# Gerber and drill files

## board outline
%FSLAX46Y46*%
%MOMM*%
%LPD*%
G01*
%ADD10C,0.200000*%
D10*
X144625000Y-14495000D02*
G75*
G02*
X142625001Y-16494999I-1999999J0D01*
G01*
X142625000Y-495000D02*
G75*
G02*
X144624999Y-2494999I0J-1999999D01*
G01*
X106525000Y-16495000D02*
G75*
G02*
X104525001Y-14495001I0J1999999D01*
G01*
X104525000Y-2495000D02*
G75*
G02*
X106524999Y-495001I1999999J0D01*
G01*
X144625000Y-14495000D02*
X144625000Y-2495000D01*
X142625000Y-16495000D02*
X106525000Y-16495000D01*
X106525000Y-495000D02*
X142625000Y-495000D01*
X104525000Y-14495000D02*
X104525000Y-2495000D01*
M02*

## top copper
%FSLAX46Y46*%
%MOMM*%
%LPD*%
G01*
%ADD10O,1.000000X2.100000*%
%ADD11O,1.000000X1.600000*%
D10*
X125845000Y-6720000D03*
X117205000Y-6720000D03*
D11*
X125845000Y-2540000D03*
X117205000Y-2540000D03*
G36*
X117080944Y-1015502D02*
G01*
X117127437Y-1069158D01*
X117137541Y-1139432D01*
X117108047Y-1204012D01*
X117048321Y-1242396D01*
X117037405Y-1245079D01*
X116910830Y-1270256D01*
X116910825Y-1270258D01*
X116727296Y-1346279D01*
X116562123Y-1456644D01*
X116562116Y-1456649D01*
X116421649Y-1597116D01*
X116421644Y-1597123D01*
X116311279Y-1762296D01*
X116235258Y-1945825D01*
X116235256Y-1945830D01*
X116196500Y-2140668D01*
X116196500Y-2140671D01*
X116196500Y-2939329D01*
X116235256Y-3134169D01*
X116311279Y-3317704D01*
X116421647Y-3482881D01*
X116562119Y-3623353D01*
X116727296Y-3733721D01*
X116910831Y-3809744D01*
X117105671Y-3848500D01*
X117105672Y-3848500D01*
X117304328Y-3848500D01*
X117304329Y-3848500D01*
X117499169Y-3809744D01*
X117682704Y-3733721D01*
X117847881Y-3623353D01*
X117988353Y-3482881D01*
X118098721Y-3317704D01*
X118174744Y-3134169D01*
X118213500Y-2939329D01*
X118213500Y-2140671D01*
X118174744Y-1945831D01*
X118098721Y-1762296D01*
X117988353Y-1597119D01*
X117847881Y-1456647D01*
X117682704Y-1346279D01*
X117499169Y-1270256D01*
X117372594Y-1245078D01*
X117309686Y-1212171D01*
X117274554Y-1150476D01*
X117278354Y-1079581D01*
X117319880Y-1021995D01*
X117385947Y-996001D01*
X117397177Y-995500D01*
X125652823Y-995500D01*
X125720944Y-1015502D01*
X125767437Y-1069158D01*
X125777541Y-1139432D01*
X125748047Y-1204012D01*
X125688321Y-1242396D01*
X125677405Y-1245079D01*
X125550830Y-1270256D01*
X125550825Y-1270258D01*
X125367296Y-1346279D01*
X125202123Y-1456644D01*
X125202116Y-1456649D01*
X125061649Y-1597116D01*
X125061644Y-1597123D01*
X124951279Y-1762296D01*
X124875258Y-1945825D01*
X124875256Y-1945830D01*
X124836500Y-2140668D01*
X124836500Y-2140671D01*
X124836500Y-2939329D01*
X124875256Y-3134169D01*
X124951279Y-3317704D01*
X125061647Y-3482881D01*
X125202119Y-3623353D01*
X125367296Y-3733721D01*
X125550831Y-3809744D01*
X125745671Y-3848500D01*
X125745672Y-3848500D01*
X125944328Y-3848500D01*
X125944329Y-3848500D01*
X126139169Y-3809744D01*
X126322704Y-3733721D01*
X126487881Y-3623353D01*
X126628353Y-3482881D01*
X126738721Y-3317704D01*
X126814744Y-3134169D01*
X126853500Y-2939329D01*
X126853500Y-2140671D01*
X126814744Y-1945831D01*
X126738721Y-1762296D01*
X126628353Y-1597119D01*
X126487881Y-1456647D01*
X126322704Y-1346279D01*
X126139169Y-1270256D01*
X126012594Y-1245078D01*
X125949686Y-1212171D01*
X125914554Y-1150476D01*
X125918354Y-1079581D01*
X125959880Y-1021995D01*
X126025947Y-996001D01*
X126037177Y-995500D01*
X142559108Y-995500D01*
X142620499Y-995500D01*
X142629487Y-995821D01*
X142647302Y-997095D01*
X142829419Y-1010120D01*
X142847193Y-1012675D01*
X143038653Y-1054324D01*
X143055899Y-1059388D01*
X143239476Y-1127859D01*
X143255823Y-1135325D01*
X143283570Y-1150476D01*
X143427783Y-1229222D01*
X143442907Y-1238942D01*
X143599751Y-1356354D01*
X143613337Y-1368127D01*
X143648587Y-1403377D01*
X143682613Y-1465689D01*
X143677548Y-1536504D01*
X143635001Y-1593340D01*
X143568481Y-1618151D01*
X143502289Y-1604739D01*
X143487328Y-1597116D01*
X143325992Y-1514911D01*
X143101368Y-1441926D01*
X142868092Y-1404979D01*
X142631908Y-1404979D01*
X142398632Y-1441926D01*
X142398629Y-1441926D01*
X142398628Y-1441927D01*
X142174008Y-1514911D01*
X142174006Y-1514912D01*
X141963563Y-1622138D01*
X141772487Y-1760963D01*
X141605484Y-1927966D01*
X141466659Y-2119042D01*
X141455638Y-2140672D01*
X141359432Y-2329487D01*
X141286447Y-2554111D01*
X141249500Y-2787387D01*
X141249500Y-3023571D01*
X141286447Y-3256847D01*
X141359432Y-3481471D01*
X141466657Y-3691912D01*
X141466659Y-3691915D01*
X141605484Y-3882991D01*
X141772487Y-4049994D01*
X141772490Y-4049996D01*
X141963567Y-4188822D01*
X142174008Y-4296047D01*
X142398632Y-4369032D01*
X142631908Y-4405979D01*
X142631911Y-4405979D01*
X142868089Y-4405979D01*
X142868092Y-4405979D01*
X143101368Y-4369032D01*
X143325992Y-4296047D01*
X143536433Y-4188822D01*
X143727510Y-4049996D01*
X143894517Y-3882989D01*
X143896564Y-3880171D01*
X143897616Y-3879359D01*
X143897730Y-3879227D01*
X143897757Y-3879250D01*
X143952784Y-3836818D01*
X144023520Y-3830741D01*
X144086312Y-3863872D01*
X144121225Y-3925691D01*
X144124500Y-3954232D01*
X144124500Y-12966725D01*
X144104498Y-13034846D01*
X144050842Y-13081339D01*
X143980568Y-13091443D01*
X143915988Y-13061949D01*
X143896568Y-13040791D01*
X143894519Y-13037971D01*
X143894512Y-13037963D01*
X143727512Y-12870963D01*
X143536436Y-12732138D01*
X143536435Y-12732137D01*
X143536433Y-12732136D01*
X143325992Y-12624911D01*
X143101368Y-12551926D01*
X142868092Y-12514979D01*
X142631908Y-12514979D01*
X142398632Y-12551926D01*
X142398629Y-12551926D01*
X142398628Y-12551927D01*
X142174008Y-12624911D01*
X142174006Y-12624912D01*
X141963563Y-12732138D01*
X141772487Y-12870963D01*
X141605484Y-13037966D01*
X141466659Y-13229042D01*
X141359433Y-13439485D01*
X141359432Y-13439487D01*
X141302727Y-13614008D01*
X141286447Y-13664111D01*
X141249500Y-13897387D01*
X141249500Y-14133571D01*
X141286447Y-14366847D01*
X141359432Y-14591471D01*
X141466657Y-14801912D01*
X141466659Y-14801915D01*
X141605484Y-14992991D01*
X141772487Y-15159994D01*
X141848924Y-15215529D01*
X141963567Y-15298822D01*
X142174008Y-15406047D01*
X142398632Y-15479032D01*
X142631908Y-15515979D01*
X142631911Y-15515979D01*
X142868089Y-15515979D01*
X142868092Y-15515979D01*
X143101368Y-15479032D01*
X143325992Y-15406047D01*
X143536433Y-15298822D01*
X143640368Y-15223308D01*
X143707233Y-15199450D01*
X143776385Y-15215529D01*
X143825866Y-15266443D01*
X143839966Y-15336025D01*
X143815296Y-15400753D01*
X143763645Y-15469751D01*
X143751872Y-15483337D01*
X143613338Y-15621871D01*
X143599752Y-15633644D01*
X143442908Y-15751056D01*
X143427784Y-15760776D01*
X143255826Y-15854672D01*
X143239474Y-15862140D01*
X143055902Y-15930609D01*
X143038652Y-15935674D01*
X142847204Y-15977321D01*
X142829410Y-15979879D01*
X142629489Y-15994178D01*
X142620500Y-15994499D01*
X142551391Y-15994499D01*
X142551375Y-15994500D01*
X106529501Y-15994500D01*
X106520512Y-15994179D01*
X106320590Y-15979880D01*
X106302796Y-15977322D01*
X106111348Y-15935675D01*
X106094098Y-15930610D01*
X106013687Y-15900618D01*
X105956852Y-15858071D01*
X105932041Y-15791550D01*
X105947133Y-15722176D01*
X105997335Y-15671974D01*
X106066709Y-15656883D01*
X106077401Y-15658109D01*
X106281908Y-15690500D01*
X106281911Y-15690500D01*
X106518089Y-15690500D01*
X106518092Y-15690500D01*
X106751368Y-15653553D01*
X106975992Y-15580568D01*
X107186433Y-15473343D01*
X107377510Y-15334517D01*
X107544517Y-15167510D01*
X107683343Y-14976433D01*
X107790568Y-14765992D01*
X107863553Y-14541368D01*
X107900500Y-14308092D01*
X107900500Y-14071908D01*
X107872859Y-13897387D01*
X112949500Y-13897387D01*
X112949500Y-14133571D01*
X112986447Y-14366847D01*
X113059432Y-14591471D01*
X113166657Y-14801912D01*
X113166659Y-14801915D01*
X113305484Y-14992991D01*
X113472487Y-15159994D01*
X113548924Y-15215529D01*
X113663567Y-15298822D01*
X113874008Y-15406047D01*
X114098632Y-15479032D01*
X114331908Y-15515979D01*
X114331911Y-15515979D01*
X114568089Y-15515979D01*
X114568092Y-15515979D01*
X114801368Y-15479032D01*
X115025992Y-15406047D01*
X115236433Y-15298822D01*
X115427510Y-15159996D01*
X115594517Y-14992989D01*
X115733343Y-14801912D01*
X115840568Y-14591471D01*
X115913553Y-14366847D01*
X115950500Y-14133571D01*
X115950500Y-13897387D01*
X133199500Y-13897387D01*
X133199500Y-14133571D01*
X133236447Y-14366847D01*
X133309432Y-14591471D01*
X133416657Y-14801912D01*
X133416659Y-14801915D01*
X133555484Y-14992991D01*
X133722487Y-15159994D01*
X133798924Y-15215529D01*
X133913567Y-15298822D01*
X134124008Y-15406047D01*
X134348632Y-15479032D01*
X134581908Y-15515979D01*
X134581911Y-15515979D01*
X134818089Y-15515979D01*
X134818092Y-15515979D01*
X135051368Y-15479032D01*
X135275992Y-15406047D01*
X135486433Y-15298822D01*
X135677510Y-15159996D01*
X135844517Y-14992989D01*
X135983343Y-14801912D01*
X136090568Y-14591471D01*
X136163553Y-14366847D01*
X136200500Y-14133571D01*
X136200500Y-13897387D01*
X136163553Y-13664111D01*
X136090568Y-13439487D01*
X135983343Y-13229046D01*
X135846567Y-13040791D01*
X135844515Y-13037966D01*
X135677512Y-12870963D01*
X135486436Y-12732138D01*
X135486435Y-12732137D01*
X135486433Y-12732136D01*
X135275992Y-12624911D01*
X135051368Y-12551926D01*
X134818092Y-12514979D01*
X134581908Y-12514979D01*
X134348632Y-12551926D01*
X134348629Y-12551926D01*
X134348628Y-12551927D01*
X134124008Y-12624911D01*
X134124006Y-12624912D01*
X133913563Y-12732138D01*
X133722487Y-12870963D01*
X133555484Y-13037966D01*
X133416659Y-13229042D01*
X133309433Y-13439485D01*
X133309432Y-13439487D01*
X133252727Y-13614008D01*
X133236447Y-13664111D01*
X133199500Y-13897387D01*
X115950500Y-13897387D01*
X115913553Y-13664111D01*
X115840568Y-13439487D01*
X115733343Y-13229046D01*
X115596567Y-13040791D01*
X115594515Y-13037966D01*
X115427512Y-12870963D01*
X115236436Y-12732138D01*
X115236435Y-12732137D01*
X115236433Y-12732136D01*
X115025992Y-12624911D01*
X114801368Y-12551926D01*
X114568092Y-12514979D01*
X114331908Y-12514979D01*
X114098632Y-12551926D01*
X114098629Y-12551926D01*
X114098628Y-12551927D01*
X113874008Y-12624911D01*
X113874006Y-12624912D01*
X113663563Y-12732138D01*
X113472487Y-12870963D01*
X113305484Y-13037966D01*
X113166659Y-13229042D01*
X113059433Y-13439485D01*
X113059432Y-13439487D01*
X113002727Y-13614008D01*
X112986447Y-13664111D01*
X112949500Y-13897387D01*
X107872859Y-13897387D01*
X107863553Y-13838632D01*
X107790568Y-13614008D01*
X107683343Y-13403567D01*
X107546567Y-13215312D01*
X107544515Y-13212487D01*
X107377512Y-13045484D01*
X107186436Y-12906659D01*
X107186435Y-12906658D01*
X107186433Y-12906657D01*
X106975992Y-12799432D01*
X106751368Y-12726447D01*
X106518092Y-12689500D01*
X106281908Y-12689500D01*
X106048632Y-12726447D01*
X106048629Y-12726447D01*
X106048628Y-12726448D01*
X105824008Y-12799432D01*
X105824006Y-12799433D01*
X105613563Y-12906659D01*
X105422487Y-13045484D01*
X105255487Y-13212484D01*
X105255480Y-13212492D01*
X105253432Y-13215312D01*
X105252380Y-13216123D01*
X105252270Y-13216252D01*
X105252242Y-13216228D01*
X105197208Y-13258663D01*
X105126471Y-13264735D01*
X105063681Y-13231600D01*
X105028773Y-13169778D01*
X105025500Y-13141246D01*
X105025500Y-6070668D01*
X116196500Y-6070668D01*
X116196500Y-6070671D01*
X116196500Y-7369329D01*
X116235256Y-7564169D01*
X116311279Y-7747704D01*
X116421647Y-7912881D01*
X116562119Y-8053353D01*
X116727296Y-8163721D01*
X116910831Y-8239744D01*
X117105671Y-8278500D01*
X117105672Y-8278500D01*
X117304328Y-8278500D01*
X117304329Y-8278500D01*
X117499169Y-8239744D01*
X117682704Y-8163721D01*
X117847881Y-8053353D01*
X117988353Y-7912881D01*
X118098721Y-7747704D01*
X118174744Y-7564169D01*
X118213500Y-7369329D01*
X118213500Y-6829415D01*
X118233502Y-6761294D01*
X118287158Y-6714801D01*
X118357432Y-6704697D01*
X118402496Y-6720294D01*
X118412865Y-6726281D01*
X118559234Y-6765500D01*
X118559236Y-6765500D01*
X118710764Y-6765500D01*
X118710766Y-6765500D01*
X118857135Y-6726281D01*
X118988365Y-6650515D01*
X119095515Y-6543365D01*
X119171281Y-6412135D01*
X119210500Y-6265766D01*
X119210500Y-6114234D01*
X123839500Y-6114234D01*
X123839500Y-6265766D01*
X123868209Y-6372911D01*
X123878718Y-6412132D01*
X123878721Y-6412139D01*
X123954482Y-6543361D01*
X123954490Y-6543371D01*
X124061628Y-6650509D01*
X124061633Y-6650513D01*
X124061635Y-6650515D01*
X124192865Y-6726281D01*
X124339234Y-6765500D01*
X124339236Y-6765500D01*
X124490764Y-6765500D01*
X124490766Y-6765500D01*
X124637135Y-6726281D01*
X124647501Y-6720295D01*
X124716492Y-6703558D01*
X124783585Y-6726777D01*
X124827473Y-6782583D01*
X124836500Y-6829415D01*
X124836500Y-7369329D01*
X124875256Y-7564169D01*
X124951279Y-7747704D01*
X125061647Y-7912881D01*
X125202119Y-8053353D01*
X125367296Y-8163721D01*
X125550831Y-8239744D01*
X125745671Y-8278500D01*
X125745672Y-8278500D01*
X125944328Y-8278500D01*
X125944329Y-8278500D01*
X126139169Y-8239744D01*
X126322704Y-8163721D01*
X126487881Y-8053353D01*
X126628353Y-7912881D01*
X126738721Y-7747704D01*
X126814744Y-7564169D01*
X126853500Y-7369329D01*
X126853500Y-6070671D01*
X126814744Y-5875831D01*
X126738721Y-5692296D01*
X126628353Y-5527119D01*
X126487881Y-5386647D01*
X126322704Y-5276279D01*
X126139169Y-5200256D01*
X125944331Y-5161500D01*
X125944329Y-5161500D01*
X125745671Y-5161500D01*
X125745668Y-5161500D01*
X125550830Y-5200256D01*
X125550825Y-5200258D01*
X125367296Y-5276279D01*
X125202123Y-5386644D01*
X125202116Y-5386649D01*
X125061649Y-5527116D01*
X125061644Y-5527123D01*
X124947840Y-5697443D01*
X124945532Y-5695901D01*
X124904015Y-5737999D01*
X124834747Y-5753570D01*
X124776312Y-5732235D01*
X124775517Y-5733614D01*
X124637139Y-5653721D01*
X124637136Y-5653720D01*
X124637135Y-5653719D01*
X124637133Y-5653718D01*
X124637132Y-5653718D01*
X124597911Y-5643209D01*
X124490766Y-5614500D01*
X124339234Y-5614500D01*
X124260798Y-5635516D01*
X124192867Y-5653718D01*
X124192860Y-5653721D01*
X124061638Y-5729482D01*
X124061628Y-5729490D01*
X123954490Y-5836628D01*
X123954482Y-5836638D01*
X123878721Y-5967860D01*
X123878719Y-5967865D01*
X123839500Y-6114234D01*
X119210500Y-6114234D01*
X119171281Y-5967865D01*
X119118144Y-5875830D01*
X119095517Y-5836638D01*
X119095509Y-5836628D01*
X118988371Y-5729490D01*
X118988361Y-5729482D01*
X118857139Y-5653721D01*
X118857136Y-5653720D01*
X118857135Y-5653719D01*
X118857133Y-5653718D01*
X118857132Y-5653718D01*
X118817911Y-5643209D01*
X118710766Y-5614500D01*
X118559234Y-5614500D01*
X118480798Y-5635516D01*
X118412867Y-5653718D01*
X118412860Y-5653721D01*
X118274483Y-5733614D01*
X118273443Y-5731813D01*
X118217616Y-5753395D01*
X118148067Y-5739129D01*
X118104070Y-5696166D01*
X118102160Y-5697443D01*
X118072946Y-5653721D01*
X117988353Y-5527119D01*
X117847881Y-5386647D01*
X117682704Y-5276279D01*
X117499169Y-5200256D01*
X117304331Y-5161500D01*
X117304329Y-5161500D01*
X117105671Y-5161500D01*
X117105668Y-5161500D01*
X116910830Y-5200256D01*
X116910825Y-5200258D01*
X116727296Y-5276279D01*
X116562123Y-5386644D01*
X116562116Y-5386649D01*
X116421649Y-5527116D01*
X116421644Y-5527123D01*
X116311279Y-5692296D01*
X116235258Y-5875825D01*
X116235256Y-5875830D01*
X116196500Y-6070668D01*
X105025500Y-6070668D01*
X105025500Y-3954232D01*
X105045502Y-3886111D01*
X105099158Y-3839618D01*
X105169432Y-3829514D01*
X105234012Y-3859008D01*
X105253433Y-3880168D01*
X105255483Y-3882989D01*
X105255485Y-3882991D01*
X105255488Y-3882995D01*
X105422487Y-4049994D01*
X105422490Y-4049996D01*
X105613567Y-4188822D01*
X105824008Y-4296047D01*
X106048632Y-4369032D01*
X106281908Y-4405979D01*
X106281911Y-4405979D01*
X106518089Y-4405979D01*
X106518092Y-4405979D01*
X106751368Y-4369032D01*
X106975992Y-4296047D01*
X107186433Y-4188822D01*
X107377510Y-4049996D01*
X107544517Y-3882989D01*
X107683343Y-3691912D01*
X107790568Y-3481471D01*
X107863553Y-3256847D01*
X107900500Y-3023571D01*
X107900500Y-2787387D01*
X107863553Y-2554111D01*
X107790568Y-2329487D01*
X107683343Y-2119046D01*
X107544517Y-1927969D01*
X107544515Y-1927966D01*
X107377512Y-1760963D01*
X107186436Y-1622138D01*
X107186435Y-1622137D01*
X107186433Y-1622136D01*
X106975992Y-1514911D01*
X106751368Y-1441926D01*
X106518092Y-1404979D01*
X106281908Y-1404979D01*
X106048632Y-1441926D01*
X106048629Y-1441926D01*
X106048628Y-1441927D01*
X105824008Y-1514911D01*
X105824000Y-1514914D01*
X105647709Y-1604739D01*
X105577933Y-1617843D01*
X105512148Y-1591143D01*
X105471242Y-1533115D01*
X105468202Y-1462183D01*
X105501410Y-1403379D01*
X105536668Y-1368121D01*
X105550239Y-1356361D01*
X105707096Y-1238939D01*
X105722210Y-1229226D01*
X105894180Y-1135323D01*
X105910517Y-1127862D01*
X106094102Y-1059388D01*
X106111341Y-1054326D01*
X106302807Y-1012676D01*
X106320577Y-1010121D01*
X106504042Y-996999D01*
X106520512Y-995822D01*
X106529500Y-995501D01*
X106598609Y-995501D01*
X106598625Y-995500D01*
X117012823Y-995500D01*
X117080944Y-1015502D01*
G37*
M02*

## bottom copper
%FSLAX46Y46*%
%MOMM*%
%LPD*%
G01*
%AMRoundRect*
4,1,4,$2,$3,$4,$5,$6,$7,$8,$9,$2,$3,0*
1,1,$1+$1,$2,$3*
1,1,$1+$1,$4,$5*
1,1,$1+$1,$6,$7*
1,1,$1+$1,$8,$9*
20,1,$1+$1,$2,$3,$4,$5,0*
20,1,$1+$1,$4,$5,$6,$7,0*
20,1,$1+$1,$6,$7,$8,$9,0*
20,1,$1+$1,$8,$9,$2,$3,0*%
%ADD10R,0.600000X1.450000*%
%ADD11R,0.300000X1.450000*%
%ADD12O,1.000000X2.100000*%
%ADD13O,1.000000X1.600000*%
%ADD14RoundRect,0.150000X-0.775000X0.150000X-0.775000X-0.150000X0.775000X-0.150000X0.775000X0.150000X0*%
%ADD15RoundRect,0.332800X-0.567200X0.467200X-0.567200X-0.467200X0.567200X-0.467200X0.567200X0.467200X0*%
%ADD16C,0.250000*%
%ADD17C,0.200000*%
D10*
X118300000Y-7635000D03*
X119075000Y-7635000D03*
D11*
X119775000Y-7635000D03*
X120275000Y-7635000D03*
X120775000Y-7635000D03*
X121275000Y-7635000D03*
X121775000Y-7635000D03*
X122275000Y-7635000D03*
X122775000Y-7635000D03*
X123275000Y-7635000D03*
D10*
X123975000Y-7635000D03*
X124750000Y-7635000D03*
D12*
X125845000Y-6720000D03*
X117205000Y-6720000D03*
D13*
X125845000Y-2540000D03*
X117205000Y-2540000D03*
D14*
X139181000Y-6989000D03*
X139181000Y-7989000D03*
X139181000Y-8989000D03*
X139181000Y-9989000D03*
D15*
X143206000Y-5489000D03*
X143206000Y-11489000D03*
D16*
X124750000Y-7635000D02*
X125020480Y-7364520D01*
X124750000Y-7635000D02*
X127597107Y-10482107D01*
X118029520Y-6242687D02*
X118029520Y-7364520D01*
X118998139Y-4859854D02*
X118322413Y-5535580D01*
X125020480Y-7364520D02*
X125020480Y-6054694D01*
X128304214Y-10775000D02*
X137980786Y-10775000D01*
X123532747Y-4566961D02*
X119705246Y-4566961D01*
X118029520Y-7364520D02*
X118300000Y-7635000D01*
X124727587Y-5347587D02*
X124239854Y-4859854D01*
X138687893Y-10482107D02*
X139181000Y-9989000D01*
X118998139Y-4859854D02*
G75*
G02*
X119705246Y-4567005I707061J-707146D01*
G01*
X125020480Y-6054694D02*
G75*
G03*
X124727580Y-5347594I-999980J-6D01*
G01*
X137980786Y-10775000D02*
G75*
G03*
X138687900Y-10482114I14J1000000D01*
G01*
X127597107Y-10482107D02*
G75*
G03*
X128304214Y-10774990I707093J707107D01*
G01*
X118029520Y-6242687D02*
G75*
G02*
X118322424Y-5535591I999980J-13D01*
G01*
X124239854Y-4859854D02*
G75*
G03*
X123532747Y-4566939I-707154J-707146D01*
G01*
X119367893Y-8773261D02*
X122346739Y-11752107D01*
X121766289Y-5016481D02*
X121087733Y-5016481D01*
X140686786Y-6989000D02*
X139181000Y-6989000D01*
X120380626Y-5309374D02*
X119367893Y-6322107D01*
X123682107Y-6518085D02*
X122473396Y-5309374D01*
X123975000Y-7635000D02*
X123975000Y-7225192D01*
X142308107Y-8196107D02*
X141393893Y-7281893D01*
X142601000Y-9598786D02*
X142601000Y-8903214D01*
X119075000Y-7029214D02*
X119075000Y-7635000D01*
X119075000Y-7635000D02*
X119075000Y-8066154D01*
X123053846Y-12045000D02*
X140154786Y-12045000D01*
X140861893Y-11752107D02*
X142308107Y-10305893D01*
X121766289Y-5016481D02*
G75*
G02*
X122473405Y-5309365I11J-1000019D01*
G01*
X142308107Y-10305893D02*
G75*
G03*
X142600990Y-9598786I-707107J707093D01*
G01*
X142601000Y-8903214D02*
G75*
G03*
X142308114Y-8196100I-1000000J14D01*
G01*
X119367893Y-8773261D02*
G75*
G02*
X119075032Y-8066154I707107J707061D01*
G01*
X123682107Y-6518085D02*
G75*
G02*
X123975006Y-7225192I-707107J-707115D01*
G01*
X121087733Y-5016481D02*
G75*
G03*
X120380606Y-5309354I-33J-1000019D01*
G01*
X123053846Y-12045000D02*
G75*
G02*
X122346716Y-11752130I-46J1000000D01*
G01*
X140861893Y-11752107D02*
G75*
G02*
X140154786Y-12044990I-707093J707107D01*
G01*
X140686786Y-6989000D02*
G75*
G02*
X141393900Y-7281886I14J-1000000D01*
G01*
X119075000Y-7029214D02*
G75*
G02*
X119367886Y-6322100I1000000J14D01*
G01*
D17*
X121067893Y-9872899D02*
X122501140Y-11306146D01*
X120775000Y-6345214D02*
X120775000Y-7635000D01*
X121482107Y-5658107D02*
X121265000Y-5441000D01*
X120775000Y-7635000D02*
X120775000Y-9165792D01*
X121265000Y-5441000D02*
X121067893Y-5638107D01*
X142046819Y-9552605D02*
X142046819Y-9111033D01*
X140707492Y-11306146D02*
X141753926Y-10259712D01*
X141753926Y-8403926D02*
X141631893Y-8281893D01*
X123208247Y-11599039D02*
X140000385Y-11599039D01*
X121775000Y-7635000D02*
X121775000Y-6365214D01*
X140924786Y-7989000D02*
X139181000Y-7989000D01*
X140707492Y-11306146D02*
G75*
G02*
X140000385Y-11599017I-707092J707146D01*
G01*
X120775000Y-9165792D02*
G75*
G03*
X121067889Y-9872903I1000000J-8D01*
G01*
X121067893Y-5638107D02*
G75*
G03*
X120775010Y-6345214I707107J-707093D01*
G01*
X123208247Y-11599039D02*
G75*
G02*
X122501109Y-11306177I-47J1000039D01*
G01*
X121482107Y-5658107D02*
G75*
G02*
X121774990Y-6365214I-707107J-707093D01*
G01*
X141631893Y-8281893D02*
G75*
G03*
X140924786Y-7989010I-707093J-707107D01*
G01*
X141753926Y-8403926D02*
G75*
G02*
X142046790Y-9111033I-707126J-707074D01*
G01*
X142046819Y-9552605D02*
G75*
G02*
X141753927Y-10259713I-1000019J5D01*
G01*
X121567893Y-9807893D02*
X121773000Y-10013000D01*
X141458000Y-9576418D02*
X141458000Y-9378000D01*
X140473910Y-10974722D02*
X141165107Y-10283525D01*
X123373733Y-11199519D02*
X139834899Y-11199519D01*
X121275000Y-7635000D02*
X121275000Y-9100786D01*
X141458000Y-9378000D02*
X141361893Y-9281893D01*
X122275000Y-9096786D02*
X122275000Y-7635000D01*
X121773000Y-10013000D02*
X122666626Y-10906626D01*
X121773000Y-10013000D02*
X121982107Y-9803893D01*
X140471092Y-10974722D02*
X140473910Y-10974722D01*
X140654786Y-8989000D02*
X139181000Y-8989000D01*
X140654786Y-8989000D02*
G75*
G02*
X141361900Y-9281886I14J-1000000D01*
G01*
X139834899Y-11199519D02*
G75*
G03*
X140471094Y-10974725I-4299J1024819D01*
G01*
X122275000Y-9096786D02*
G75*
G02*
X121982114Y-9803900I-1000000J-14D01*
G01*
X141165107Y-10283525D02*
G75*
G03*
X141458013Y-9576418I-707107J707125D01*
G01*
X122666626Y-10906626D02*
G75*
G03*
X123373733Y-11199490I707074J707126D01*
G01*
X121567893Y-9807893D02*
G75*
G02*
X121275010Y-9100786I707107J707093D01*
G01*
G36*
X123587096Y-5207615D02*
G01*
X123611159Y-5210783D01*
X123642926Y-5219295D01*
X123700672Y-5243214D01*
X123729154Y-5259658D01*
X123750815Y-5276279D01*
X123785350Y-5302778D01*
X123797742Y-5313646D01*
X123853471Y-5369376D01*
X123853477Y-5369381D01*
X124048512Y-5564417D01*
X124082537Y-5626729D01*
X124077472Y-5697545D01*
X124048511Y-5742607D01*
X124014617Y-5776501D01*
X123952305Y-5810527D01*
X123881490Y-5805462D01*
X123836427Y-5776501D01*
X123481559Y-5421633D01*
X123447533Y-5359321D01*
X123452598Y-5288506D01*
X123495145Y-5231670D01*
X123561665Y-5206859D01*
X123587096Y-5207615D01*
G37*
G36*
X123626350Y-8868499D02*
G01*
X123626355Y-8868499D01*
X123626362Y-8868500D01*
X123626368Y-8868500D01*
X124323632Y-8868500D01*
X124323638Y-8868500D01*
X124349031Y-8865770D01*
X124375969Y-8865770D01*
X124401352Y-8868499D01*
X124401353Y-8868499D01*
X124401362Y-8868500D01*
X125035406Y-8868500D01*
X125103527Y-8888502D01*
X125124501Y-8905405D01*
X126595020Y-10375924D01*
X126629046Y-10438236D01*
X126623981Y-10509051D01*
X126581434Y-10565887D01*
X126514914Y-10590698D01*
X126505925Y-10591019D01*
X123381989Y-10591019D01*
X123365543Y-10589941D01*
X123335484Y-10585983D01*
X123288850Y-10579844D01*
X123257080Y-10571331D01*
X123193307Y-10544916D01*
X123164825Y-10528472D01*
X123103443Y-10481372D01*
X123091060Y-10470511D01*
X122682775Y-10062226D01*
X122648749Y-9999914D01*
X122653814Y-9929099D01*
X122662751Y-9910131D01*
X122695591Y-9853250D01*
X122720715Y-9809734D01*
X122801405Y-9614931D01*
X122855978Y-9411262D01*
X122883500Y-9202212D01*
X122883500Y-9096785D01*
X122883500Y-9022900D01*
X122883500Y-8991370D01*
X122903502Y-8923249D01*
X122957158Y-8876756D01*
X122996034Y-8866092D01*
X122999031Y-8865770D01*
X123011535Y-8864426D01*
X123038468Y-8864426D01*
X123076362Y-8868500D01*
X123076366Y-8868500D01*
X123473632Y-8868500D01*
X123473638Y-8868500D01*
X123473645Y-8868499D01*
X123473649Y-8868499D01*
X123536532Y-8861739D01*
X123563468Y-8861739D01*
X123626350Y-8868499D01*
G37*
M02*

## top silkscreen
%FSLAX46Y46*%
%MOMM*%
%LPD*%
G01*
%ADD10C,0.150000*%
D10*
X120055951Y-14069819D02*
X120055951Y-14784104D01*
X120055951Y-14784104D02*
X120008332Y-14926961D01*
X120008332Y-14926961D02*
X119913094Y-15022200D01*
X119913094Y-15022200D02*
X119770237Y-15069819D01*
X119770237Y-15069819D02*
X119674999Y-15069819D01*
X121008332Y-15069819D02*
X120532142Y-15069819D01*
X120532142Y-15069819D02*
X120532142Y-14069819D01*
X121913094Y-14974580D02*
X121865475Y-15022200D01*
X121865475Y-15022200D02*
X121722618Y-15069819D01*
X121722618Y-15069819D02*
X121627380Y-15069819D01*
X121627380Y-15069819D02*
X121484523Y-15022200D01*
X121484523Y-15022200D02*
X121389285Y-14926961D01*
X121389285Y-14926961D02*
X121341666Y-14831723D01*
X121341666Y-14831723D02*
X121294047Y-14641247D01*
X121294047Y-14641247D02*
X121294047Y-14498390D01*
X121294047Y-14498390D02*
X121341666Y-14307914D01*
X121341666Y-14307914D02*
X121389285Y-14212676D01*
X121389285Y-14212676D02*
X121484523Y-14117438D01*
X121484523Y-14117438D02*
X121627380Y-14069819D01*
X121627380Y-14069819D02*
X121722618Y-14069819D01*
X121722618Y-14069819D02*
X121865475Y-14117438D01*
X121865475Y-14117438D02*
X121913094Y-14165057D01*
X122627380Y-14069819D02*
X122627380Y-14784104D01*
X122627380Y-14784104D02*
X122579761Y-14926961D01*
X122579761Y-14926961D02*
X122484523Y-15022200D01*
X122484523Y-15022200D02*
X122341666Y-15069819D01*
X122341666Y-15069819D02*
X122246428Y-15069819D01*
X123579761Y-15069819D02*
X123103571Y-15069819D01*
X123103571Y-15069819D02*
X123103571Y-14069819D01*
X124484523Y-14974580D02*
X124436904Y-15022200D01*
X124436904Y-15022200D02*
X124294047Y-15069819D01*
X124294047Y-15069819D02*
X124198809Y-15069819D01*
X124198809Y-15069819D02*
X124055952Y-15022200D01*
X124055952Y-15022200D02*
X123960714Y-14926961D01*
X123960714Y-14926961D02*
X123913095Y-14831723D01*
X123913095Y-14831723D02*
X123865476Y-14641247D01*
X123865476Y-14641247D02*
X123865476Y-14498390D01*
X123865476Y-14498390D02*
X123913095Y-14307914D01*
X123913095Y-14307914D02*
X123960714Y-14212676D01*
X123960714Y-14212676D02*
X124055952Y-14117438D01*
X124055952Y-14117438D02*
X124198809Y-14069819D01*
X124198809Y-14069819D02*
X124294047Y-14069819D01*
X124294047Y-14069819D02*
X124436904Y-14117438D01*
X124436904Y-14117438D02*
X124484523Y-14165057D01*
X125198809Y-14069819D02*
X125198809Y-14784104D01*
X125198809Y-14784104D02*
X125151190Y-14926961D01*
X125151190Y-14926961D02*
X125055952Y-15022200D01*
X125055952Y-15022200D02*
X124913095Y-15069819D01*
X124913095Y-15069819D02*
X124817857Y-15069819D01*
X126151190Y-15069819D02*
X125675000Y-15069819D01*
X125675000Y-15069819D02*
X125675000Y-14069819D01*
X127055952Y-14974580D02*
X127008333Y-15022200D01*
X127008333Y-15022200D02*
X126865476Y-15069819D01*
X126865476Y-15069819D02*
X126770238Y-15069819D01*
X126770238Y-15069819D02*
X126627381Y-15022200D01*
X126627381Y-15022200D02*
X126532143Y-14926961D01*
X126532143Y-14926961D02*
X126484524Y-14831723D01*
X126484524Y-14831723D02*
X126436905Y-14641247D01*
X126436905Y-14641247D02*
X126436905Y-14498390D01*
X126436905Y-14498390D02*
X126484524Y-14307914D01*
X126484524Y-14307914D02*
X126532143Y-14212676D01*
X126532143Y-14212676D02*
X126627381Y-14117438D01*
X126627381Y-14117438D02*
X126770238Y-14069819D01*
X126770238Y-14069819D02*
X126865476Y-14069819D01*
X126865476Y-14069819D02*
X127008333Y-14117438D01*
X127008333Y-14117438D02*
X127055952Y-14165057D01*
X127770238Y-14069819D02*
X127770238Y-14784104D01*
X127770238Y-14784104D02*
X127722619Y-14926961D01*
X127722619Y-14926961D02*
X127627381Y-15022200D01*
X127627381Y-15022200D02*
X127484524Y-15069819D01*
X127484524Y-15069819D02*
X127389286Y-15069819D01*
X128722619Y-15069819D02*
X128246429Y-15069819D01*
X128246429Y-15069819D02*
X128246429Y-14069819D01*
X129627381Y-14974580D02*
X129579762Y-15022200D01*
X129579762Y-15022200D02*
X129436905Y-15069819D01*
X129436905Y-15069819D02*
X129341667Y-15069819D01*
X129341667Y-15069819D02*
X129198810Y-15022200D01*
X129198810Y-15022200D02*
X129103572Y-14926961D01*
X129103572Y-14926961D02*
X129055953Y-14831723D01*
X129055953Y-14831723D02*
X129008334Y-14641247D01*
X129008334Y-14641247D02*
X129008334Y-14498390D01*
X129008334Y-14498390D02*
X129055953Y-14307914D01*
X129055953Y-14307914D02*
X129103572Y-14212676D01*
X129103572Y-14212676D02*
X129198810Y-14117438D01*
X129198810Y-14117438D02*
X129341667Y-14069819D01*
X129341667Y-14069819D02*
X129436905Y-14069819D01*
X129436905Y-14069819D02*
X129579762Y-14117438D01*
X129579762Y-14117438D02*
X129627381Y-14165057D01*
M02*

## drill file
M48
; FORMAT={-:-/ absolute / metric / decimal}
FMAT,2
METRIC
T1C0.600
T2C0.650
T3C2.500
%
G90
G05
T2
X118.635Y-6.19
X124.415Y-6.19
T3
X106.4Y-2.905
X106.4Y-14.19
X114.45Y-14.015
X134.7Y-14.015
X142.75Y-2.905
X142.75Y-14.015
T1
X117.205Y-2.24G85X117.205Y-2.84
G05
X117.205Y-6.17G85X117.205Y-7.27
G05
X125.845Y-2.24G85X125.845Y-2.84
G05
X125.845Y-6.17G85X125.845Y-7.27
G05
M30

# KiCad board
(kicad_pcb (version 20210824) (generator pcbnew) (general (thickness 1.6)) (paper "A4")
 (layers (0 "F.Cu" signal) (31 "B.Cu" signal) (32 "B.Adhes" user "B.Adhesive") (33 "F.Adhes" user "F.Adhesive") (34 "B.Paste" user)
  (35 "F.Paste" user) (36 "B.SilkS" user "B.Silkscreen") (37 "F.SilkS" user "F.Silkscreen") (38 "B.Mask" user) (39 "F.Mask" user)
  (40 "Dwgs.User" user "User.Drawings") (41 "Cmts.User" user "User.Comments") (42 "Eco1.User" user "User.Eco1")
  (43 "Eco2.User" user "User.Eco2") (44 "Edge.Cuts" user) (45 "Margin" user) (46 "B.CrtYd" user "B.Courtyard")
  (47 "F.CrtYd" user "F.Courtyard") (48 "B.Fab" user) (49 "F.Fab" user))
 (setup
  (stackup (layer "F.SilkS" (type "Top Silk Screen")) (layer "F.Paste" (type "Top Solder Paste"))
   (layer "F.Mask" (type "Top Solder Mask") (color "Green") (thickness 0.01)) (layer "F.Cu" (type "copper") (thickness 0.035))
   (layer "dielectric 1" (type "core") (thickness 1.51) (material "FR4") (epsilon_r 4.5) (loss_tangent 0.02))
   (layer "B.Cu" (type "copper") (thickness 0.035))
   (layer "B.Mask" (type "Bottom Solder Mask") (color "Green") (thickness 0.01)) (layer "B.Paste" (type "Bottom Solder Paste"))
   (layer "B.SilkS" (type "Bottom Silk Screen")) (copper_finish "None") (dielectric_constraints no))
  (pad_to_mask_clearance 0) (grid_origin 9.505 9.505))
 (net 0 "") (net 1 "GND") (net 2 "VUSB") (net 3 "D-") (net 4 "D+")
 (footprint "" (layer "F.Cu") (at 136.255 14.205)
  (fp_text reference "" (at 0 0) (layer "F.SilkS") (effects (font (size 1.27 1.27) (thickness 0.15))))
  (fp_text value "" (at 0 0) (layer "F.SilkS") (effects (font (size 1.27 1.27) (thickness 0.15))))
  (pad "" np_thru_hole circle (at -1.555 -0.189521) (size 2.5 2.5) (drill 2.5) (layers F&B.Cu *.Mask)))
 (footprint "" (layer "F.Cu") (at 94.555 1.535)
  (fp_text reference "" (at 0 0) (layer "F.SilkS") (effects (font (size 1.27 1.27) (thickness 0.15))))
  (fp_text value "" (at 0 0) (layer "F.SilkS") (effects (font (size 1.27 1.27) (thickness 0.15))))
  (pad "" np_thru_hole circle (at 11.845 1.370479) (size 2.5 2.5) (drill 2.5) (layers F&B.Cu *.Mask)))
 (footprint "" (layer "F.Cu") (at 147.015 3.065)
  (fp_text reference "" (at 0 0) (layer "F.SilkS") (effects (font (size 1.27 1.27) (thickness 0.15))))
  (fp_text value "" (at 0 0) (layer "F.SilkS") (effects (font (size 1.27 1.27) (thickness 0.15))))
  (pad "" np_thru_hole circle (at -4.265 -0.159521) (size 2.5 2.5) (drill 2.5) (layers F&B.Cu *.Mask)))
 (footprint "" (layer "F.Cu") (at 94.295 7.445633)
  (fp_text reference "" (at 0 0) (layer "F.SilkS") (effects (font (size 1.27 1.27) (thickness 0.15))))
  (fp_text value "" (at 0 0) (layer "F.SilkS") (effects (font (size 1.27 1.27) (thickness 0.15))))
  (pad "" np_thru_hole circle (at 12.105 6.744367) (size 2.5 2.5) (drill 2.5) (layers F&B.Cu *.Mask)))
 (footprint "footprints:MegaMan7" (layer "F.Cu") (at 109.650838 8.415023)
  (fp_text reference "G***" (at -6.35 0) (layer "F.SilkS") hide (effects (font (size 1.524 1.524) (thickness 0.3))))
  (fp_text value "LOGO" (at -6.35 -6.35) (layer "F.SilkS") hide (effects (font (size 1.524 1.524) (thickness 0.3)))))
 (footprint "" (layer "F.Cu") (at 112.225 13.965)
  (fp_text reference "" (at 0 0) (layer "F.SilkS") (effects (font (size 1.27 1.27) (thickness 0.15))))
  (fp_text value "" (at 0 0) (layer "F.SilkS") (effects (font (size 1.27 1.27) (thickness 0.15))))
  (pad "" np_thru_hole circle (at 2.225 0.050479) (size 2.5 2.5) (drill 2.5) (layers F&B.Cu *.Mask)))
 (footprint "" (layer "F.Cu") (at 130.75 14.19)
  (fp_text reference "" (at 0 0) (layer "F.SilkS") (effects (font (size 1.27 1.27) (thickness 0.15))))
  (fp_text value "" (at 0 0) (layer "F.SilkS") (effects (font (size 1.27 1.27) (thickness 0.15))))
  (pad "" np_thru_hole circle (at 12 -0.174521) (size 2.5 2.5) (drill 2.5) (layers F&B.Cu *.Mask)))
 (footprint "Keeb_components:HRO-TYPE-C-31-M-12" (layer "B.Cu") (at 121.525 -0.06)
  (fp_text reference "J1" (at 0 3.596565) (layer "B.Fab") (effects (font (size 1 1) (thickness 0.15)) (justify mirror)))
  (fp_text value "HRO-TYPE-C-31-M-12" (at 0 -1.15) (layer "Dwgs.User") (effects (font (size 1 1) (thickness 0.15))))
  (pad "" np_thru_hole circle locked (at -2.89 6.25) (size 0.65 0.65) (drill 0.65) (layers *.Cu *.Mask))
  (pad "" np_thru_hole circle locked (at 2.89 6.25) (size 0.65 0.65) (drill 0.65) (layers *.Cu *.Mask))
  (pad "1" smd rect locked (at -3.225 7.695) (size 0.6 1.45) (layers "B.Cu" "B.Paste" "B.Mask") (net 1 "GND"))
  (pad "2" smd rect locked (at -2.45 7.695) (size 0.6 1.45) (layers "B.Cu" "B.Paste" "B.Mask") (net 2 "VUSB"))
  (pad "3" smd rect locked (at -1.75 7.695) (size 0.3 1.45) (layers "B.Cu" "B.Paste" "B.Mask"))
  (pad "4" smd rect locked (at -1.25 7.695) (size 0.3 1.45) (layers "B.Cu" "B.Paste" "B.Mask"))
  (pad "5" smd rect locked (at -0.75 7.695) (size 0.3 1.45) (layers "B.Cu" "B.Paste" "B.Mask") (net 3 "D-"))
  (pad "6" smd rect locked (at -0.25 7.695) (size 0.3 1.45) (layers "B.Cu" "B.Paste" "B.Mask") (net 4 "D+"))
  (pad "7" smd rect locked (at 0.25 7.695) (size 0.3 1.45) (layers "B.Cu" "B.Paste" "B.Mask") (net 3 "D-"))
  (pad "8" smd rect locked (at 0.75 7.695) (size 0.3 1.45) (layers "B.Cu" "B.Paste" "B.Mask") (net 4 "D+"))
  (pad "9" smd rect locked (at 1.25 7.695) (size 0.3 1.45) (layers "B.Cu" "B.Paste" "B.Mask"))
  (pad "10" smd rect locked (at 1.75 7.695) (size 0.3 1.45) (layers "B.Cu" "B.Paste" "B.Mask"))
  (pad "11" smd rect locked (at 2.45 7.695) (size 0.6 1.45) (layers "B.Cu" "B.Paste" "B.Mask") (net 2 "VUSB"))
  (pad "12" smd rect locked (at 3.225 7.695) (size 0.6 1.45) (layers "B.Cu" "B.Paste" "B.Mask") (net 1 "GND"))
  (pad "13" thru_hole oval locked (at 4.32 6.78) (size 1 2.1) (drill oval 0.6 1.7) (layers *.Cu *.Mask))
  (pad "13" thru_hole oval locked (at -4.32 6.78) (size 1 2.1) (drill oval 0.6 1.7) (layers *.Cu *.Mask))
  (pad "13" thru_hole oval locked (at 4.32 2.6) (size 1 1.6) (drill oval 0.6 1.2) (layers *.Cu *.Mask))
  (pad "13" thru_hole oval locked (at -4.32 2.6) (size 1 1.6) (drill oval 0.6 1.2) (layers *.Cu *.Mask)))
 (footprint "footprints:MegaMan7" (layer "B.Cu") (at 109.650838 8.39588 180)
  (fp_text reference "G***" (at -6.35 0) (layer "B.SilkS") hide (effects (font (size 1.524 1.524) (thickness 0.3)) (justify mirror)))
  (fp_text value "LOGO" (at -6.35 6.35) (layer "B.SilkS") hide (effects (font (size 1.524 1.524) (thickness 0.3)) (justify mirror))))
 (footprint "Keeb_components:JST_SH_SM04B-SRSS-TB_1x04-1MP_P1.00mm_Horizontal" (layer "B.Cu") (at 141.331 8.489 -90)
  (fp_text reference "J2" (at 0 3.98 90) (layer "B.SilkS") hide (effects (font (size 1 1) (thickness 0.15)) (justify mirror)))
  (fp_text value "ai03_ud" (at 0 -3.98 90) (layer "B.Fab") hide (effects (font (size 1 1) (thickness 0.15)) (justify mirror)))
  (pad "1" smd roundrect locked (at -1.5 2.15 270) (size 0.6 1.85) (layers "B.Cu" "B.Paste" "B.Mask") (roundrect_rratio 0.25) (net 2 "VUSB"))
  (pad "2" smd roundrect locked (at -0.5 2.15 270) (size 0.6 1.85) (layers "B.Cu" "B.Paste" "B.Mask") (roundrect_rratio 0.25) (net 3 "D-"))
  (pad "3" smd roundrect locked (at 0.5 2.15 270) (size 0.6 1.85) (layers "B.Cu" "B.Paste" "B.Mask") (roundrect_rratio 0.25) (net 4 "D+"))
  (pad "4" smd roundrect locked (at 1.5 2.15 270) (size 0.6 1.85) (layers "B.Cu" "B.Paste" "B.Mask") (roundrect_rratio 0.25) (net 1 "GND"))
  (pad "MP" smd roundrect locked (at -3 -1.875 270) (size 1.6 1.8) (layers "B.Cu" "B.Paste" "B.Mask") (roundrect_rratio 0.208))
  (pad "MP" smd roundrect locked (at 3 -1.875 270) (size 1.6 1.8) (layers "B.Cu" "B.Paste" "B.Mask") (roundrect_rratio 0.208)))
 (gr_arc (start 142.625001 14.495) (end 144.625 14.495) (angle 90) (layer "Edge.Cuts") (width 0.2))
 (gr_arc (start 142.625 2.494999) (end 142.625 0.495) (angle 90) (layer "Edge.Cuts") (width 0.2))
 (gr_arc (start 106.525 14.495001) (end 106.525 16.495) (angle 90) (layer "Edge.Cuts") (width 0.2))
 (gr_arc (start 106.524999 2.495) (end 104.525 2.495) (angle 90) (layer "Edge.Cuts") (width 0.2))
 (gr_line (start 144.625 14.495) (end 144.625 2.495) (layer "Edge.Cuts") (width 0.2))
 (gr_line (start 142.625 16.495) (end 106.525 16.495) (layer "Edge.Cuts") (width 0.2))
 (gr_line (start 106.525 0.495) (end 142.625 0.495) (layer "Edge.Cuts") (width 0.2))
 (gr_line (start 104.525 14.495) (end 104.525 2.495) (layer "Edge.Cuts") (width 0.2))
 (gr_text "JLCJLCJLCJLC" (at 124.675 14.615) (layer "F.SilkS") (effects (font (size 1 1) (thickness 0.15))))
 (segment (start 124.75 7.635) (end 125.02048 7.36452) (width 0.25) (layer "B.Cu") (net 1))
 (segment (start 124.75 7.635) (end 127.597107 10.482107) (width 0.25) (layer "B.Cu") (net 1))
 (segment (start 118.02952 6.242687) (end 118.02952 7.36452) (width 0.25) (layer "B.Cu") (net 1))
 (segment (start 118.998139 4.859854) (end 118.322413 5.53558) (width 0.25) (layer "B.Cu") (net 1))
 (segment (start 125.02048 7.36452) (end 125.02048 6.054694) (width 0.25) (layer "B.Cu") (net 1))
 (segment (start 128.304214 10.775) (end 137.980786 10.775) (width 0.25) (layer "B.Cu") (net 1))
 (segment (start 123.532747 4.566961) (end 119.705246 4.566961) (width 0.25) (layer "B.Cu") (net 1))
 (segment (start 118.02952 7.36452) (end 118.3 7.635) (width 0.25) (layer "B.Cu") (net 1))
 (segment (start 124.727587 5.347587) (end 124.239854 4.859854) (width 0.25) (layer "B.Cu") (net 1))
 (segment (start 138.687893 10.482107) (end 139.181 9.989) (width 0.25) (layer "B.Cu") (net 1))
 (arc (start 118.998139 4.859854) (mid 119.322562 4.643081) (end 119.705246 4.566961) (width 0.25) (layer "B.Cu") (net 1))
 (arc (start 125.02048 6.054694) (mid 124.94436 5.672011) (end 124.727587 5.347587) (width 0.25) (layer "B.Cu") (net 1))
 (arc (start 137.980786 10.775) (mid 138.363469 10.69888) (end 138.687893 10.482107) (width 0.25) (layer "B.Cu") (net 1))
 (arc (start 127.597107 10.482107) (mid 127.92153 10.69888) (end 128.304214 10.775) (width 0.25) (layer "B.Cu") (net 1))
 (arc (start 118.02952 6.242687) (mid 118.10564 5.860004) (end 118.322413 5.53558) (width 0.25) (layer "B.Cu") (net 1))
 (arc (start 124.239854 4.859854) (mid 123.915431 4.643081) (end 123.532747 4.566961) (width 0.25) (layer "B.Cu") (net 1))
 (segment (start 119.367893 8.773261) (end 122.346739 11.752107) (width 0.25) (layer "B.Cu") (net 2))
 (segment (start 121.766289 5.016481) (end 121.087733 5.016481) (width 0.25) (layer "B.Cu") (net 2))
 (segment (start 140.686786 6.989) (end 139.181 6.989) (width 0.25) (layer "B.Cu") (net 2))
 (segment (start 120.380626 5.309374) (end 119.367893 6.322107) (width 0.25) (layer "B.Cu") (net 2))
 (segment (start 123.682107 6.518085) (end 122.473396 5.309374) (width 0.25) (layer "B.Cu") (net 2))
 (segment (start 123.975 7.635) (end 123.975 7.225192) (width 0.25) (layer "B.Cu") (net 2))
 (segment (start 142.308107 8.196107) (end 141.393893 7.281893) (width 0.25) (layer "B.Cu") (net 2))
 (segment (start 142.601 9.598786) (end 142.601 8.903214) (width 0.25) (layer "B.Cu") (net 2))
 (segment (start 119.075 7.029214) (end 119.075 7.635) (width 0.25) (layer "B.Cu") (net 2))
 (segment (start 119.075 7.635) (end 119.075 8.066154) (width 0.25) (layer "B.Cu") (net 2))
 (segment (start 123.053846 12.045) (end 140.154786 12.045) (width 0.25) (layer "B.Cu") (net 2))
 (segment (start 140.861893 11.752107) (end 142.308107 10.305893) (width 0.25) (layer "B.Cu") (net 2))
 (arc (start 121.766289 5.016481) (mid 122.148972 5.092601) (end 122.473396 5.309374) (width 0.25) (layer "B.Cu") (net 2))
 (arc (start 142.308107 10.305893) (mid 142.52488 9.98147) (end 142.601 9.598786) (width 0.25) (layer "B.Cu") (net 2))
 (arc (start 142.601 8.903214) (mid 142.52488 8.520531) (end 142.308107 8.196107) (width 0.25) (layer "B.Cu") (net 2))
 (arc (start 119.367893 8.773261) (mid 119.15112 8.448838) (end 119.075 8.066154) (width 0.25) (layer "B.Cu") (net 2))
 (arc (start 123.682107 6.518085) (mid 123.89888 6.842508) (end 123.975 7.225192) (width 0.25) (layer "B.Cu") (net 2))
 (arc (start 121.087733 5.016481) (mid 120.70505 5.092601) (end 120.380626 5.309374) (width 0.25) (layer "B.Cu") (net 2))
 (arc (start 123.053846 12.045) (mid 122.671163 11.96888) (end 122.346739 11.752107) (width 0.25) (layer "B.Cu") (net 2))
 (arc (start 140.861893 11.752107) (mid 140.53747 11.96888) (end 140.154786 12.045) (width 0.25) (layer "B.Cu") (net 2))
 (arc (start 140.686786 6.989) (mid 141.069469 7.06512) (end 141.393893 7.281893) (width 0.25) (layer "B.Cu") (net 2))
 (arc (start 119.075 7.029214) (mid 119.15112 6.646531) (end 119.367893 6.322107) (width 0.25) (layer "B.Cu") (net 2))
 (segment (start 121.067893 9.872899) (end 122.50114 11.306146) (width 0.2) (layer "B.Cu") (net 3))
 (segment (start 120.775 6.345214) (end 120.775 7.635) (width 0.2) (layer "B.Cu") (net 3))
 (segment (start 121.482107 5.658107) (end 121.265 5.441) (width 0.2) (layer "B.Cu") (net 3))
 (segment (start 120.775 7.635) (end 120.775 9.165792) (width 0.2) (layer "B.Cu") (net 3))
 (segment (start 121.265 5.441) (end 121.067893 5.638107) (width 0.2) (layer "B.Cu") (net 3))
 (segment (start 142.046819 9.552605) (end 142.046819 9.111033) (width 0.2) (layer "B.Cu") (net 3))
 (segment (start 140.707492 11.306146) (end 141.753926 10.259712) (width 0.2) (layer "B.Cu") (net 3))
 (segment (start 141.753926 8.403926) (end 141.631893 8.281893) (width 0.2) (layer "B.Cu") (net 3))
 (segment (start 123.208247 11.599039) (end 140.000385 11.599039) (width 0.2) (layer "B.Cu") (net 3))
 (segment (start 121.775 7.635) (end 121.775 6.365214) (width 0.2) (layer "B.Cu") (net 3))
 (segment (start 140.924786 7.989) (end 139.181 7.989) (width 0.2) (layer "B.Cu") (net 3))
 (arc (start 140.707492 11.306146) (mid 140.383069 11.522919) (end 140.000385 11.599039) (width 0.2) (layer "B.Cu") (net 3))
 (arc (start 120.775 9.165792) (mid 120.85112 9.548475) (end 121.067893 9.872899) (width 0.2) (layer "B.Cu") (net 3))
 (arc (start 121.067893 5.638107) (mid 120.85112 5.96253) (end 120.775 6.345214) (width 0.2) (layer "B.Cu") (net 3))
 (arc (start 123.208247 11.599039) (mid 122.825564 11.522919) (end 122.50114 11.306146) (width 0.2) (layer "B.Cu") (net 3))
 (arc (start 121.482107 5.658107) (mid 121.69888 5.98253) (end 121.775 6.365214) (width 0.2) (layer "B.Cu") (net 3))
 (arc (start 141.631893 8.281893) (mid 141.30747 8.06512) (end 140.924786 7.989) (width 0.2) (layer "B.Cu") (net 3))
 (arc (start 141.753926 8.403926) (mid 141.970699 8.728349) (end 142.046819 9.111033) (width 0.2) (layer "B.Cu") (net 3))
 (arc (start 142.046819 9.552605) (mid 141.970699 9.935288) (end 141.753926 10.259712) (width 0.2) (layer "B.Cu") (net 3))
 (segment (start 121.567893 9.807893) (end 121.773 10.013) (width 0.2) (layer "B.Cu") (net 4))
 (segment (start 141.458 9.576418) (end 141.458 9.378) (width 0.2) (layer "B.Cu") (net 4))
 (segment (start 140.47391 10.974722) (end 141.165107 10.283525) (width 0.2) (layer "B.Cu") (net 4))
 (segment (start 123.373733 11.199519) (end 139.834899 11.199519) (width 0.2) (layer "B.Cu") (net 4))
 (segment (start 121.275 7.635) (end 121.275 9.100786) (width 0.2) (layer "B.Cu") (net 4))
 (segment (start 141.458 9.378) (end 141.361893 9.281893) (width 0.2) (layer "B.Cu") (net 4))
 (segment (start 122.275 9.096786) (end 122.275 7.635) (width 0.2) (layer "B.Cu") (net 4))
 (segment (start 121.773 10.013) (end 122.666626 10.906626) (width 0.2) (layer "B.Cu") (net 4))
 (segment (start 121.773 10.013) (end 121.982107 9.803893) (width 0.2) (layer "B.Cu") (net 4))
 (segment (start 140.471092 10.974722) (end 140.47391 10.974722) (width 0.2) (layer "B.Cu") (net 4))
 (segment (start 140.654786 8.989) (end 139.181 8.989) (width 0.2) (layer "B.Cu") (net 4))
 (arc (start 140.654786 8.989) (mid 141.037469 9.06512) (end 141.361893 9.281893) (width 0.2) (layer "B.Cu") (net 4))
 (arc (start 139.834899 11.199519) (mid 140.171789 11.141063) (end 140.471092 10.974722) (width 0.2) (layer "B.Cu") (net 4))
 (arc (start 122.275 9.096786) (mid 122.19888 9.479469) (end 121.982107 9.803893) (width 0.2) (layer "B.Cu") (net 4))
 (arc (start 141.165107 10.283525) (mid 141.38188 9.959102) (end 141.458 9.576418) (width 0.2) (layer "B.Cu") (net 4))
 (arc (start 122.666626 10.906626) (mid 122.991049 11.123399) (end 123.373733 11.199519) (width 0.2) (layer "B.Cu") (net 4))
 (arc (start 121.567893 9.807893) (mid 121.35112 9.48347) (end 121.275 9.100786) (width 0.2) (layer "B.Cu") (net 4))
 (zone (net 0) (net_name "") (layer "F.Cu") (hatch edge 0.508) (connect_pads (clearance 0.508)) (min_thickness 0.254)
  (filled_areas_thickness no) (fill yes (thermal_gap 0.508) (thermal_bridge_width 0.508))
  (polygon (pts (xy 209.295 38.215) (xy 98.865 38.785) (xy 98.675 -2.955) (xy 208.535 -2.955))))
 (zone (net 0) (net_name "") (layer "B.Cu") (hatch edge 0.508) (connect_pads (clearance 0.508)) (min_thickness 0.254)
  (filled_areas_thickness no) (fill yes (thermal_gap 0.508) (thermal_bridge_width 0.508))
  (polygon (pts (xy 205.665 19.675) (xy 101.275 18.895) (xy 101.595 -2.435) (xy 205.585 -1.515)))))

